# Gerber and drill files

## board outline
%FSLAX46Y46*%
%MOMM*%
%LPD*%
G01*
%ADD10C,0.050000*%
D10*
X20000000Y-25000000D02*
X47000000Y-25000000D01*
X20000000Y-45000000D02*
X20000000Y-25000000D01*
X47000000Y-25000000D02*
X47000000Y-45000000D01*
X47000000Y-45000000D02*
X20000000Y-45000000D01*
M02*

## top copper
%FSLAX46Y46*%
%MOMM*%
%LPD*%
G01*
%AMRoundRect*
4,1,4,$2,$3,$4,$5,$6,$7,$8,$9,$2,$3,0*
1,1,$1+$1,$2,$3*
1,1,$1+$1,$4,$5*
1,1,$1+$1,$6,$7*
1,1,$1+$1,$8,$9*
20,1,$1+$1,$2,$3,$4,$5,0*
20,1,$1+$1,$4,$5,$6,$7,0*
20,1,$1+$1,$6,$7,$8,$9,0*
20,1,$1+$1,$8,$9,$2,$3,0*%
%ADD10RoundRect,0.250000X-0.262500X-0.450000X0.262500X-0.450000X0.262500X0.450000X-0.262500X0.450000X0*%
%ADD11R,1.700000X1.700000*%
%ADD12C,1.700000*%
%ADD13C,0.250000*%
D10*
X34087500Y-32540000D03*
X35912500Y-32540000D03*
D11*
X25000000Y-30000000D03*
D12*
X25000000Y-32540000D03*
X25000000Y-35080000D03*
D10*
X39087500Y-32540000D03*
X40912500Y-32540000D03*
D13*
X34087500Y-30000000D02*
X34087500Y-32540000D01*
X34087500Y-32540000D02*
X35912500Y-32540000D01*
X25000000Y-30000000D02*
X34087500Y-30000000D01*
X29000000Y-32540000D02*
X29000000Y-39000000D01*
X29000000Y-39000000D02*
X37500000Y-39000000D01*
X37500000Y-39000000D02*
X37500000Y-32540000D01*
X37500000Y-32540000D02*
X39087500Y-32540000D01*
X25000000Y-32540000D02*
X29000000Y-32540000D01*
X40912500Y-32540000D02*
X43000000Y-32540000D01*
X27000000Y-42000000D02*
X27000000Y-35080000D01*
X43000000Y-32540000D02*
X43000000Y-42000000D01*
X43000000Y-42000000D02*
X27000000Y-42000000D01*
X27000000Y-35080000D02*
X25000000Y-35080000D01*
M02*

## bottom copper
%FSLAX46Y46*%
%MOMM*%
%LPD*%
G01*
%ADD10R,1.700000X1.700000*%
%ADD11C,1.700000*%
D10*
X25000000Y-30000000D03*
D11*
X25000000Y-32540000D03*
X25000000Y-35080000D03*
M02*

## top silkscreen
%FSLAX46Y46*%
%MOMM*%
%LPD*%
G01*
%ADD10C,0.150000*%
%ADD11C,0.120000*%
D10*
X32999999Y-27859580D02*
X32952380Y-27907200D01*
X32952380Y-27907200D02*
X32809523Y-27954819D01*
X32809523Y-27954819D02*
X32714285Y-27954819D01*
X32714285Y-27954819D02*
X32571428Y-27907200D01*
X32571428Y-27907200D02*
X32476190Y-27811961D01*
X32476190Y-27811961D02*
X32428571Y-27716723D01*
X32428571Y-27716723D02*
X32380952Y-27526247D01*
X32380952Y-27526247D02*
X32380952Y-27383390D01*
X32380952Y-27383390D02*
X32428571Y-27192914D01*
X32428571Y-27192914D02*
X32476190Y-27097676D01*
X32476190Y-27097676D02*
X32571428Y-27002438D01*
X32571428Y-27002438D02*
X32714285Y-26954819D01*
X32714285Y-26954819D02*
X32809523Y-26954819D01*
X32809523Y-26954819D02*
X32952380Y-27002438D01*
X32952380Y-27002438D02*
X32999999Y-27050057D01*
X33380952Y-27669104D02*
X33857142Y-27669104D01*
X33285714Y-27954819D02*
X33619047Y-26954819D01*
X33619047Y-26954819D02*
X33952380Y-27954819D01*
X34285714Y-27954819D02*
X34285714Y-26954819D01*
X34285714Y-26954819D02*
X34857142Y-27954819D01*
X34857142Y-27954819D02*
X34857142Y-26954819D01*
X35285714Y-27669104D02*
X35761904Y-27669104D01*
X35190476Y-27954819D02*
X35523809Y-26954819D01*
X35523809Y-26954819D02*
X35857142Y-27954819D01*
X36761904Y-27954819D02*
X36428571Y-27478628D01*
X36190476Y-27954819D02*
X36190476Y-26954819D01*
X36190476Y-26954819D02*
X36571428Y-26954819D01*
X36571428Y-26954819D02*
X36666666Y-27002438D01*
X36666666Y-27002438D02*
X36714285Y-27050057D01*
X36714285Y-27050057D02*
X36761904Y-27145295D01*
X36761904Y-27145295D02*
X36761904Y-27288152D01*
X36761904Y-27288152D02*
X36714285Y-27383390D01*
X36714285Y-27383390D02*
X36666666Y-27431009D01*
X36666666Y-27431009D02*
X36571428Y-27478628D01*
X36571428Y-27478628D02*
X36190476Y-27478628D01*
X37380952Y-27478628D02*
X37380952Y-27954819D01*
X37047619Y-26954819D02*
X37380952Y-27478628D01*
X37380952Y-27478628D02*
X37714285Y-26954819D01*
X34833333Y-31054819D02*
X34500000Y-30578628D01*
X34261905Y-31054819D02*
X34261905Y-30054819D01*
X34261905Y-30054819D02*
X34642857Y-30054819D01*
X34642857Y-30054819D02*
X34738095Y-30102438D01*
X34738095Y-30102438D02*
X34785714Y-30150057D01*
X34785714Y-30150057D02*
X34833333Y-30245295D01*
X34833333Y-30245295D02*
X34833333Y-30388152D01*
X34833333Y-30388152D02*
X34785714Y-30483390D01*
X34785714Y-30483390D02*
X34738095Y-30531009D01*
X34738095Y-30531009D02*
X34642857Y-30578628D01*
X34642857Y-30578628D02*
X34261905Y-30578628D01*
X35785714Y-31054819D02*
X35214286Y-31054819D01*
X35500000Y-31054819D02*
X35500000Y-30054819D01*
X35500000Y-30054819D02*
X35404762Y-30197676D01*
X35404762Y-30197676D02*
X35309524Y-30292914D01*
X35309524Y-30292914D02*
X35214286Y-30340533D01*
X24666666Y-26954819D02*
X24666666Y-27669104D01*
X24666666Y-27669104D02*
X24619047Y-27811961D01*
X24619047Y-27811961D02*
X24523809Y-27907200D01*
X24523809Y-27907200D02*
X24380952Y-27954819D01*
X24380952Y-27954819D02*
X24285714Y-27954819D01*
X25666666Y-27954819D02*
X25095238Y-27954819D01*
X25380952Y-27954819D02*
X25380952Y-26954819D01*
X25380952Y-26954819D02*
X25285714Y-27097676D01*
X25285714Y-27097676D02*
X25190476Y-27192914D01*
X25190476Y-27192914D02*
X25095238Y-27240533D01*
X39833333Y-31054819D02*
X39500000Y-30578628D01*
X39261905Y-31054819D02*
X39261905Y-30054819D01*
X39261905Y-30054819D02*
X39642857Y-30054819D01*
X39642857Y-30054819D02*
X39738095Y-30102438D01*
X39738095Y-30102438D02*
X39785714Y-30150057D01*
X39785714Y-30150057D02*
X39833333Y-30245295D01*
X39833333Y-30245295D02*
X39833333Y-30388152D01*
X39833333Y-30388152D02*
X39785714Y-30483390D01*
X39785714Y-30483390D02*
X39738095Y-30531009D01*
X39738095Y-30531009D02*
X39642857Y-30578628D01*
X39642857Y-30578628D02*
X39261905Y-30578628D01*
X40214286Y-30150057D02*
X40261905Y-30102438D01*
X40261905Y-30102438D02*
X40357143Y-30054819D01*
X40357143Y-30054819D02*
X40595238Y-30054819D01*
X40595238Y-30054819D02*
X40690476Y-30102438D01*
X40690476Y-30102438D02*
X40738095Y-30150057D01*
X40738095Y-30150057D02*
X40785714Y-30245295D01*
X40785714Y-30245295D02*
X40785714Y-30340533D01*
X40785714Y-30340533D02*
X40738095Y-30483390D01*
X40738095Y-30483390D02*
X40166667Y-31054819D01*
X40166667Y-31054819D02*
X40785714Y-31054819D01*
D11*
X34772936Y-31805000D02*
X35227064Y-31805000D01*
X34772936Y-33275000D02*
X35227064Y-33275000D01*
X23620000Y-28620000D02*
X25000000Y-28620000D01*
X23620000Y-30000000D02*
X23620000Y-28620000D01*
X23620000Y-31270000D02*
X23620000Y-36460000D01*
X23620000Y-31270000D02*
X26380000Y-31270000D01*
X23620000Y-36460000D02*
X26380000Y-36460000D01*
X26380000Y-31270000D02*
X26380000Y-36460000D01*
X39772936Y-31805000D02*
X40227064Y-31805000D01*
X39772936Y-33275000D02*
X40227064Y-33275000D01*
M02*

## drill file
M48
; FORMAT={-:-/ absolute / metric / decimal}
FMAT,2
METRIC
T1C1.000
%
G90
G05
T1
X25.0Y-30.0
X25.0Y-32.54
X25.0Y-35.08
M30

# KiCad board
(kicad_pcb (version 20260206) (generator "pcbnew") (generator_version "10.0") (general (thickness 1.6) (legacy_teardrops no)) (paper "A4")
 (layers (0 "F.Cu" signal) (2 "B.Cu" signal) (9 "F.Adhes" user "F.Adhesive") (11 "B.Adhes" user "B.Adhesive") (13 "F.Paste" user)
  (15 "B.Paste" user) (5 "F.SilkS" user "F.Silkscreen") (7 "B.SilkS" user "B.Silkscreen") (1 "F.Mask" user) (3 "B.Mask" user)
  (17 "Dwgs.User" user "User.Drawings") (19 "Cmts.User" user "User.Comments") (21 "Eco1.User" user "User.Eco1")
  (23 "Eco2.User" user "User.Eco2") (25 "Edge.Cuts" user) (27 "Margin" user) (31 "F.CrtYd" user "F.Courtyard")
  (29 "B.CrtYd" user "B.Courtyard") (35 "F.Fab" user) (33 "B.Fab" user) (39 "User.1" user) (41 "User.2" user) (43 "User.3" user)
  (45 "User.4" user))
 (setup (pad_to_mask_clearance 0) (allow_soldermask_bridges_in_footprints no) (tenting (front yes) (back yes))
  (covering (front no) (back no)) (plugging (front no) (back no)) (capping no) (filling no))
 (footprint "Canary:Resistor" (layer "F.Cu") (at 35 32.54)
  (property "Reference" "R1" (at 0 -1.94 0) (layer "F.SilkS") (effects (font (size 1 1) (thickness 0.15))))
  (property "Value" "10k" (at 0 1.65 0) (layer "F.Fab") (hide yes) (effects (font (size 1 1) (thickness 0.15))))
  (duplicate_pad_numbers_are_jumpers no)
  (fp_line (start -0.227064 -0.735) (end 0.227064 -0.735) (stroke (width 0.12) (type solid)) (layer "F.SilkS"))
  (fp_line (start -0.227064 0.735) (end 0.227064 0.735) (stroke (width 0.12) (type solid)) (layer "F.SilkS"))
  (pad "1" smd roundrect (at -0.9125 0) (size 1.025 1.4) (layers "F.Cu" "F.Mask" "F.Paste") (roundrect_rratio 0.243902) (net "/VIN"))
  (pad "2" smd roundrect (at 0.9125 0) (size 1.025 1.4) (layers "F.Cu" "F.Mask" "F.Paste") (roundrect_rratio 0.243902) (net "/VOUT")))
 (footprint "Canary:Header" (layer "F.Cu") (at 25 30)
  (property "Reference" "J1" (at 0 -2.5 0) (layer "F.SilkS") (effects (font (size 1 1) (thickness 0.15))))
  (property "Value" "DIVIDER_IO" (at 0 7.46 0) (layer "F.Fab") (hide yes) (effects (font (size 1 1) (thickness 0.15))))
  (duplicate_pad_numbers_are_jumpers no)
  (fp_line (start -1.38 -1.38) (end 0 -1.38) (stroke (width 0.12) (type solid)) (layer "F.SilkS"))
  (fp_line (start -1.38 0) (end -1.38 -1.38) (stroke (width 0.12) (type solid)) (layer "F.SilkS"))
  (fp_line (start -1.38 1.27) (end -1.38 6.46) (stroke (width 0.12) (type solid)) (layer "F.SilkS"))
  (fp_line (start -1.38 1.27) (end 1.38 1.27) (stroke (width 0.12) (type solid)) (layer "F.SilkS"))
  (fp_line (start -1.38 6.46) (end 1.38 6.46) (stroke (width 0.12) (type solid)) (layer "F.SilkS"))
  (fp_line (start 1.38 1.27) (end 1.38 6.46) (stroke (width 0.12) (type solid)) (layer "F.SilkS"))
  (pad "1" thru_hole rect (at 0 0) (size 1.7 1.7) (drill 1) (layers "*.Cu" "*.Mask") (remove_unused_layers no) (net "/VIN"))
  (pad "2" thru_hole circle (at 0 2.54) (size 1.7 1.7) (drill 1) (layers "*.Cu" "*.Mask") (remove_unused_layers no) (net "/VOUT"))
  (pad "3" thru_hole circle (at 0 5.08) (size 1.7 1.7) (drill 1) (layers "*.Cu" "*.Mask") (remove_unused_layers no) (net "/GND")))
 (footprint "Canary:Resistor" (layer "F.Cu") (at 40 32.54)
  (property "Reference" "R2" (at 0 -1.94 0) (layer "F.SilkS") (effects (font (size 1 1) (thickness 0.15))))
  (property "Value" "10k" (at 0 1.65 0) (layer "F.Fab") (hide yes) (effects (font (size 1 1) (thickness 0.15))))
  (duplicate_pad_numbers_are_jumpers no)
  (fp_line (start -0.227064 -0.735) (end 0.227064 -0.735) (stroke (width 0.12) (type solid)) (layer "F.SilkS"))
  (fp_line (start -0.227064 0.735) (end 0.227064 0.735) (stroke (width 0.12) (type solid)) (layer "F.SilkS"))
  (pad "1" smd roundrect (at -0.9125 0) (size 1.025 1.4) (layers "F.Cu" "F.Mask" "F.Paste") (roundrect_rratio 0.243902) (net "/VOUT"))
  (pad "2" smd roundrect (at 0.9125 0) (size 1.025 1.4) (layers "F.Cu" "F.Mask" "F.Paste") (roundrect_rratio 0.243902) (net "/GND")))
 (gr_line (start 20 25) (end 47 25) (stroke (width 0.05) (type default)) (layer "Edge.Cuts"))
 (gr_line (start 20 45) (end 20 25) (stroke (width 0.05) (type default)) (layer "Edge.Cuts"))
 (gr_line (start 47 25) (end 47 45) (stroke (width 0.05) (type default)) (layer "Edge.Cuts"))
 (gr_line (start 47 45) (end 20 45) (stroke (width 0.05) (type default)) (layer "Edge.Cuts"))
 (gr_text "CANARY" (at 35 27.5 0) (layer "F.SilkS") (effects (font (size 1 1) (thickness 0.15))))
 (segment (start 34.0875 30) (end 34.0875 32.54) (width 0.25) (layer "F.Cu") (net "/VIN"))
 (segment (start 34.0875 32.54) (end 35.9125 32.54) (width 0.25) (layer "F.Cu") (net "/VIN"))
 (segment (start 25 30) (end 34.0875 30) (width 0.25) (layer "F.Cu") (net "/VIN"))
 (segment (start 29 32.54) (end 29 39) (width 0.25) (layer "F.Cu") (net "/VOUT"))
 (segment (start 29 39) (end 37.5 39) (width 0.25) (layer "F.Cu") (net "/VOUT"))
 (segment (start 37.5 39) (end 37.5 32.54) (width 0.25) (layer "F.Cu") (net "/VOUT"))
 (segment (start 37.5 32.54) (end 39.0875 32.54) (width 0.25) (layer "F.Cu") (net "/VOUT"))
 (segment (start 25 32.54) (end 29 32.54) (width 0.25) (layer "F.Cu") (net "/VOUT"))
 (segment (start 40.9125 32.54) (end 43 32.54) (width 0.25) (layer "F.Cu") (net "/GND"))
 (segment (start 27 42) (end 27 35.08) (width 0.25) (layer "F.Cu") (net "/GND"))
 (segment (start 43 32.54) (end 43 42) (width 0.25) (layer "F.Cu") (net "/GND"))
 (segment (start 43 42) (end 27 42) (width 0.25) (layer "F.Cu") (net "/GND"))
 (segment (start 27 35.08) (end 25 35.08) (width 0.25) (layer "F.Cu") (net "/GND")))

